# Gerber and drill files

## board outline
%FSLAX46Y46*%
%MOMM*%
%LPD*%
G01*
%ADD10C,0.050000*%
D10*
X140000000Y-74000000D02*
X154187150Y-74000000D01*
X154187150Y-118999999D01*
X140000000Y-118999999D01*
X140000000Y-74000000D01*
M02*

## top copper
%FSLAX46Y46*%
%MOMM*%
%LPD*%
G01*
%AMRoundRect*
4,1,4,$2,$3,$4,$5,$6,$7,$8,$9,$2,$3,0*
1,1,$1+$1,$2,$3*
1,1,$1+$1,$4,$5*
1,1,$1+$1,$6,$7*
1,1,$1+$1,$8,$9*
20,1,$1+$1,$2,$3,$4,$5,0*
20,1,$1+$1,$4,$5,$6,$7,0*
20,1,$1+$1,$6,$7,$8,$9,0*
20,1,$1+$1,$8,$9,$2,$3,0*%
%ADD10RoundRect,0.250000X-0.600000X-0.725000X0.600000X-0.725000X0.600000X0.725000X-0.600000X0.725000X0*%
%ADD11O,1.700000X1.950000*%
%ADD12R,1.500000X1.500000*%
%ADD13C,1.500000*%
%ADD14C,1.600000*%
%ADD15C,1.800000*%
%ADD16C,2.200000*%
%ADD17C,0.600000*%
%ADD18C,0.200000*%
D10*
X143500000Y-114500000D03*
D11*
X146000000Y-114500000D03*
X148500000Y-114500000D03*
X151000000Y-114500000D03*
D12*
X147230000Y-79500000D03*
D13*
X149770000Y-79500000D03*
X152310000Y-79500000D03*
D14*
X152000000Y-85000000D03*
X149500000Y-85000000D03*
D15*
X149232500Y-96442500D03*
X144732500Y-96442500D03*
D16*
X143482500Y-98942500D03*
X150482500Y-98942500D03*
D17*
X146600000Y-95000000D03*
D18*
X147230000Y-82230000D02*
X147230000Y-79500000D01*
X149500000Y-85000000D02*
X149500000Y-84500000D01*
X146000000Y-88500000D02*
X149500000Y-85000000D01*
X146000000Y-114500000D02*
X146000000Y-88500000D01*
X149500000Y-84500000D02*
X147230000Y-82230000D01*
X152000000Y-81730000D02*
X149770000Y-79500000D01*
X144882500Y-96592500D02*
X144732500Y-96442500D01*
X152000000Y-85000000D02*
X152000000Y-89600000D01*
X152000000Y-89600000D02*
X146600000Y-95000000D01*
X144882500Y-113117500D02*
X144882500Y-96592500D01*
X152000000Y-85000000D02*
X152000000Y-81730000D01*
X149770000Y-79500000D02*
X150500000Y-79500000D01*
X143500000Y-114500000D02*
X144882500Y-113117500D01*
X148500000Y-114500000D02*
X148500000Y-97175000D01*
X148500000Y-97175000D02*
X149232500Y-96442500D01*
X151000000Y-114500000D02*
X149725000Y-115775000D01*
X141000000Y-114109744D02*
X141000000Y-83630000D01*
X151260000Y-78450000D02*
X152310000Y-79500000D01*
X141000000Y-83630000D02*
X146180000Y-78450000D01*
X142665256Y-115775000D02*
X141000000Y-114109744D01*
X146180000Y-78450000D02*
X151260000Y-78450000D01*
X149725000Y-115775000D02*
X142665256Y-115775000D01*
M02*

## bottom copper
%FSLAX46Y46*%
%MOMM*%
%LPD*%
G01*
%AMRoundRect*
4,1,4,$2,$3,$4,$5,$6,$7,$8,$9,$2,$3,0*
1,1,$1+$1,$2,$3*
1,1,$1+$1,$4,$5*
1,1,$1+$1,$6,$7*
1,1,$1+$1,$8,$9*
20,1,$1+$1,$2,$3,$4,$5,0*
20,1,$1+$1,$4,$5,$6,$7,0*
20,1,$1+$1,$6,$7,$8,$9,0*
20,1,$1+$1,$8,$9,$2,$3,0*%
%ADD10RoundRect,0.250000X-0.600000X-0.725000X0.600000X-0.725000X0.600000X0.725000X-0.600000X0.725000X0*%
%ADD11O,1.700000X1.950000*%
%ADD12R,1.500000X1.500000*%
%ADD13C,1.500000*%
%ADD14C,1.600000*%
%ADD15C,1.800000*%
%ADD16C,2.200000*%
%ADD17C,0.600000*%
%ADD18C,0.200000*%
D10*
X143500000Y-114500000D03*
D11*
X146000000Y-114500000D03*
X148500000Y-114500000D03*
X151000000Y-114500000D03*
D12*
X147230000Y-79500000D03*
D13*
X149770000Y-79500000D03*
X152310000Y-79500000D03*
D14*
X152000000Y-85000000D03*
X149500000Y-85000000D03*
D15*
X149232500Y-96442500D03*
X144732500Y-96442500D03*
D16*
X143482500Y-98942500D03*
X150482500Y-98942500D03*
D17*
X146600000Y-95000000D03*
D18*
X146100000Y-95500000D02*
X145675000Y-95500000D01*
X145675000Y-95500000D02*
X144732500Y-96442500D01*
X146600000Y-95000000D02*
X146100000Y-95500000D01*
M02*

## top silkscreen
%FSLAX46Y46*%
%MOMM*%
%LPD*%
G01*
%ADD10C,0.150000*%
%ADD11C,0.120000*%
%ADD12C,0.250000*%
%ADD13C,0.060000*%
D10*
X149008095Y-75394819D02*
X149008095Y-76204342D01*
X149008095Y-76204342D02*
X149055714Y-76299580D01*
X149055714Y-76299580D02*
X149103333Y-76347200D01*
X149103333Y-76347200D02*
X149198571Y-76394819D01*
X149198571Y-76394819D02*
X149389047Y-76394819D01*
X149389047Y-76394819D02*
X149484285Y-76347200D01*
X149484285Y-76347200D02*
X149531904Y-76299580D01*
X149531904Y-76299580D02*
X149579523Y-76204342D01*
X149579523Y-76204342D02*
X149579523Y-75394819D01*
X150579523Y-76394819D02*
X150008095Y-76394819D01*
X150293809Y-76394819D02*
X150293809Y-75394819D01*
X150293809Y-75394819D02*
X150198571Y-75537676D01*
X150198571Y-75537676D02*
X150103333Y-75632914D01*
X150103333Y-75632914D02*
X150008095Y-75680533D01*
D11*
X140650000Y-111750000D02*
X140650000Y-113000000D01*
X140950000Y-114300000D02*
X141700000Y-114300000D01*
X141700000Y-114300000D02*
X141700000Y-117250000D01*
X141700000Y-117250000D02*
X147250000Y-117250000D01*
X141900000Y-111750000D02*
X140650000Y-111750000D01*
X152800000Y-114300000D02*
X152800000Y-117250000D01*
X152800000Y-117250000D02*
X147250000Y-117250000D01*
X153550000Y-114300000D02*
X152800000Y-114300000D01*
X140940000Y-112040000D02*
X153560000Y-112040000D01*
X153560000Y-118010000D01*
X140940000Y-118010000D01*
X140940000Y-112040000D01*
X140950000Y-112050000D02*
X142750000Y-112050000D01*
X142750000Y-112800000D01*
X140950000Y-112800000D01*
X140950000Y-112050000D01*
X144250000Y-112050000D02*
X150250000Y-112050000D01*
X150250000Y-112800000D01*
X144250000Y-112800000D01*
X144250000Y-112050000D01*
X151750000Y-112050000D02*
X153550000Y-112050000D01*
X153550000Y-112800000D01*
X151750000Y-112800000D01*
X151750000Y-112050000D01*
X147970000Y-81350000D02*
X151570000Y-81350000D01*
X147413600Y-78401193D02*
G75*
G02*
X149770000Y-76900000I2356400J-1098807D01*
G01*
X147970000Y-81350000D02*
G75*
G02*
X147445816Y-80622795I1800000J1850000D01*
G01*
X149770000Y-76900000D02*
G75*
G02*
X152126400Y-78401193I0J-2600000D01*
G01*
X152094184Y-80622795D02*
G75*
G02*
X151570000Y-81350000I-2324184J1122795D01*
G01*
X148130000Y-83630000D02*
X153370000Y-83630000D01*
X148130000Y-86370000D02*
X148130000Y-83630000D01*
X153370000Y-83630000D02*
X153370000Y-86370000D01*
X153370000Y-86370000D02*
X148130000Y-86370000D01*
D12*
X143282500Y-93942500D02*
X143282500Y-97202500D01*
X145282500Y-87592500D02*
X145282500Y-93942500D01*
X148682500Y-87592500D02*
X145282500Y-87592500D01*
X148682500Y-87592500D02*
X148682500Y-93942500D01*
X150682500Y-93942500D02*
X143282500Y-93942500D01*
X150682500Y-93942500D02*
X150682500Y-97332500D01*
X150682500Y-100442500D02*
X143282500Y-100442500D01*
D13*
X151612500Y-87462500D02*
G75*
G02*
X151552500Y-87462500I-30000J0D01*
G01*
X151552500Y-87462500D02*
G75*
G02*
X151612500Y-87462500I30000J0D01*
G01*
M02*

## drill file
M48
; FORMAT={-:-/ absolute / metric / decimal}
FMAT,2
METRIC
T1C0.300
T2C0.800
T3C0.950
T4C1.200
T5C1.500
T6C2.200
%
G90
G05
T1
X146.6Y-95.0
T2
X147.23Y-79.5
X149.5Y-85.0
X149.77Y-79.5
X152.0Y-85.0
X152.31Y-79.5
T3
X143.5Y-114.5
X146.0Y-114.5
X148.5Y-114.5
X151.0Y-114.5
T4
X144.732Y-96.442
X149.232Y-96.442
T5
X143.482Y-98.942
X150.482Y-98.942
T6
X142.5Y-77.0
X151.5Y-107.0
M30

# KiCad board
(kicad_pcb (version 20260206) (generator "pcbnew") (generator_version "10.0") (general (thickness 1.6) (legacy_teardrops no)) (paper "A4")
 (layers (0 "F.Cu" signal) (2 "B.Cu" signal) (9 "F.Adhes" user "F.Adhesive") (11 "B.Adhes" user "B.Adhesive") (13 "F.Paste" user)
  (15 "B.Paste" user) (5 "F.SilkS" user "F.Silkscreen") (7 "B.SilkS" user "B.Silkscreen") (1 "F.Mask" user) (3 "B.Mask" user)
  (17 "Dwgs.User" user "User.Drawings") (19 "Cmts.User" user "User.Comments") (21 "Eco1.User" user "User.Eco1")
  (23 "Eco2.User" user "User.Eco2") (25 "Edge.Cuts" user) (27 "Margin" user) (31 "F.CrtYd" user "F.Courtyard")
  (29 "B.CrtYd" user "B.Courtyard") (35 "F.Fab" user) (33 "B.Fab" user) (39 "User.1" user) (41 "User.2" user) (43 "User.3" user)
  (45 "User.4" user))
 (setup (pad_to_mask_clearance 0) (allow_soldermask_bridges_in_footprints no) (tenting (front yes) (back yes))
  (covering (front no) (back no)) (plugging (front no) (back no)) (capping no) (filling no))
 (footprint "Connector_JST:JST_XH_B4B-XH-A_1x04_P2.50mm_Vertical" (layer "F.Cu") (at 143.5 114.5)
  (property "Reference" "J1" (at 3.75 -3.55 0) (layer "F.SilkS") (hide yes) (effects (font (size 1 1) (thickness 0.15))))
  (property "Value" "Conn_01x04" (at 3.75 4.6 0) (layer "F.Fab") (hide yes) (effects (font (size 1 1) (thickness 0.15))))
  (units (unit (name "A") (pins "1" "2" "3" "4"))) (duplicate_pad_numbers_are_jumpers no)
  (fp_line (start -2.85 -2.75) (end -2.85 -1.5) (stroke (width 0.12) (type solid)) (layer "F.SilkS"))
  (fp_line (start -2.55 -0.2) (end -1.8 -0.2) (stroke (width 0.12) (type solid)) (layer "F.SilkS"))
  (fp_line (start -1.8 -0.2) (end -1.8 2.75) (stroke (width 0.12) (type solid)) (layer "F.SilkS"))
  (fp_line (start -1.8 2.75) (end 3.75 2.75) (stroke (width 0.12) (type solid)) (layer "F.SilkS"))
  (fp_line (start -1.6 -2.75) (end -2.85 -2.75) (stroke (width 0.12) (type solid)) (layer "F.SilkS"))
  (fp_line (start 9.3 -0.2) (end 9.3 2.75) (stroke (width 0.12) (type solid)) (layer "F.SilkS"))
  (fp_line (start 9.3 2.75) (end 3.75 2.75) (stroke (width 0.12) (type solid)) (layer "F.SilkS"))
  (fp_line (start 10.05 -0.2) (end 9.3 -0.2) (stroke (width 0.12) (type solid)) (layer "F.SilkS"))
  (fp_rect (start -2.56 -2.46) (end 10.06 3.51) (stroke (width 0.12) (type solid)) (fill no) (layer "F.SilkS"))
  (fp_rect (start -2.55 -2.45) (end -0.75 -1.7) (stroke (width 0.12) (type solid)) (fill no) (layer "F.SilkS"))
  (fp_rect (start 0.75 -2.45) (end 6.75 -1.7) (stroke (width 0.12) (type solid)) (fill no) (layer "F.SilkS"))
  (fp_rect (start 8.25 -2.45) (end 10.05 -1.7) (stroke (width 0.12) (type solid)) (fill no) (layer "F.SilkS"))
  (pad "1" thru_hole roundrect (at 0 0) (size 1.7 1.95) (drill 0.95) (layers "*.Cu" "*.Mask") (remove_unused_layers no)
   (roundrect_rratio 0.147059) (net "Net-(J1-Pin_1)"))
  (pad "2" thru_hole oval (at 2.5 0) (size 1.7 1.95) (drill 0.95) (layers "*.Cu" "*.Mask") (remove_unused_layers no) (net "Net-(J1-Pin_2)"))
  (pad "3" thru_hole oval (at 5 0) (size 1.7 1.95) (drill 0.95) (layers "*.Cu" "*.Mask") (remove_unused_layers no) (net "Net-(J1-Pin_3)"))
  (pad "4" thru_hole oval (at 7.5 0) (size 1.7 1.95) (drill 0.95) (layers "*.Cu" "*.Mask") (remove_unused_layers no) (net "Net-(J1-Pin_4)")))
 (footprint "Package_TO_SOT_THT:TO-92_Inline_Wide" (layer "F.Cu") (at 147.23 79.5)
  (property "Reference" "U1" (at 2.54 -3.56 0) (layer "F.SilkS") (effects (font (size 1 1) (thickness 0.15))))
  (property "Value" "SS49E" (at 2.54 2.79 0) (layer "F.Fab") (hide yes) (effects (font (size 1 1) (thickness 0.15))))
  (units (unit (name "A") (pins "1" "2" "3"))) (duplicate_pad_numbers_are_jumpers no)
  (fp_line (start 0.74 1.85) (end 4.34 1.85) (stroke (width 0.12) (type solid)) (layer "F.SilkS"))
  (fp_arc (start 0.1836 -1.098807) (mid 1.143021 -2.192817) (end 2.54 -2.6) (stroke (width 0.12) (type solid)) (layer "F.SilkS"))
  (fp_arc (start 0.74 1.85) (mid 0.446097 1.509328) (end 0.215816 1.122795) (stroke (width 0.12) (type solid)) (layer "F.SilkS"))
  (fp_arc (start 2.54 -2.6) (mid 3.936979 -2.192818) (end 4.8964 -1.098807) (stroke (width 0.12) (type solid)) (layer "F.SilkS"))
  (fp_arc (start 4.864184 1.122795) (mid 4.633903 1.509328) (end 4.34 1.85) (stroke (width 0.12) (type solid)) (layer "F.SilkS"))
  (pad "1" thru_hole rect (at 0 0) (size 1.5 1.5) (drill 0.8) (layers "*.Cu" "*.Mask") (remove_unused_layers no) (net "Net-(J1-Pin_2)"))
  (pad "2" thru_hole circle (at 2.54 0) (size 1.5 1.5) (drill 0.8) (layers "*.Cu" "*.Mask") (remove_unused_layers no) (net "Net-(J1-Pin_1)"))
  (pad "3" thru_hole circle (at 5.08 0) (size 1.5 1.5) (drill 0.8) (layers "*.Cu" "*.Mask") (remove_unused_layers no) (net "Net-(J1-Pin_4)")))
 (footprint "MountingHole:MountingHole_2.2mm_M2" (layer "F.Cu") (at 142.5 77)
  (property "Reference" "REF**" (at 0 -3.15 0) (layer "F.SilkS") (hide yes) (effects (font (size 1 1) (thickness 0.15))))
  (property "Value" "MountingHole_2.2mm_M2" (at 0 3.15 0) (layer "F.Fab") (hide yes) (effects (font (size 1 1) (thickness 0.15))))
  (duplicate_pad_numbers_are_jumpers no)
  (pad "" np_thru_hole circle (at 0 0) (size 2.2 2.2) (drill 2.2) (layers "*.Cu" "*.Mask")))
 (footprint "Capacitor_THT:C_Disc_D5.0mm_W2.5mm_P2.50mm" (layer "F.Cu") (at 152 85 180)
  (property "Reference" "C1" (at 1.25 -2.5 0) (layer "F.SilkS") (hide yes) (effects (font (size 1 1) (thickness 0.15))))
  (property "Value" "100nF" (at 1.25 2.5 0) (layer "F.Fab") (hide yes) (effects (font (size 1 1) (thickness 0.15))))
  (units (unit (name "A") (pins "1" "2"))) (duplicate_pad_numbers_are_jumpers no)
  (fp_line (start 3.87 1.37) (end -1.37 1.37) (stroke (width 0.12) (type solid)) (layer "F.SilkS"))
  (fp_line (start 3.87 -1.37) (end 3.87 1.37) (stroke (width 0.12) (type solid)) (layer "F.SilkS"))
  (fp_line (start -1.37 1.37) (end -1.37 -1.37) (stroke (width 0.12) (type solid)) (layer "F.SilkS"))
  (fp_line (start -1.37 -1.37) (end 3.87 -1.37) (stroke (width 0.12) (type solid)) (layer "F.SilkS"))
  (pad "1" thru_hole circle (at 0 0 180) (size 1.6 1.6) (drill 0.8) (layers "*.Cu" "*.Mask") (remove_unused_layers no)
   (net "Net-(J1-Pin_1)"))
  (pad "2" thru_hole circle (at 2.5 0 180) (size 1.6 1.6) (drill 0.8) (layers "*.Cu" "*.Mask") (remove_unused_layers no)
   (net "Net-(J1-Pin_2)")))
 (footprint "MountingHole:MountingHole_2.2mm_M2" (layer "F.Cu") (at 151.5 107)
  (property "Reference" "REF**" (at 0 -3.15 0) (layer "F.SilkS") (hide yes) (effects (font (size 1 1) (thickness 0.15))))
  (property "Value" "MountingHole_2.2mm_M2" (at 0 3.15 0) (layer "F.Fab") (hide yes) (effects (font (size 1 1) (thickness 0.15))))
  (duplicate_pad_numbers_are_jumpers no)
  (pad "" np_thru_hole circle (at 0 0) (size 2.2 2.2) (drill 2.2) (layers "*.Cu" "*.Mask")))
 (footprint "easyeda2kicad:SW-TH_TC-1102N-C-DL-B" (layer "F.Cu") (at 146.9825 97.6925 180)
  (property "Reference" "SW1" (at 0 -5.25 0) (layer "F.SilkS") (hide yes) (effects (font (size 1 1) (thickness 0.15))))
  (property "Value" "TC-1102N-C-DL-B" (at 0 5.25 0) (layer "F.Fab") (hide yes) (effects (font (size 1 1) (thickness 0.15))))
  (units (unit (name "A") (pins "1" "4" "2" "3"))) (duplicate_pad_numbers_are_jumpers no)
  (fp_line (start 3.7 3.75) (end 3.7 0.49) (stroke (width 0.25) (type solid)) (layer "F.SilkS"))
  (fp_line (start 1.7 10.1) (end 1.7 3.75) (stroke (width 0.25) (type solid)) (layer "F.SilkS"))
  (fp_line (start -1.7 10.1) (end 1.7 10.1) (stroke (width 0.25) (type solid)) (layer "F.SilkS"))
  (fp_line (start -1.7 10.1) (end -1.7 3.75) (stroke (width 0.25) (type solid)) (layer "F.SilkS"))
  (fp_line (start -3.7 3.75) (end 3.7 3.75) (stroke (width 0.25) (type solid)) (layer "F.SilkS"))
  (fp_line (start -3.7 3.75) (end -3.7 0.36) (stroke (width 0.25) (type solid)) (layer "F.SilkS"))
  (fp_line (start -3.7 -2.75) (end 3.7 -2.75) (stroke (width 0.25) (type solid)) (layer "F.SilkS"))
  (fp_circle (center -4.6 10.23) (end -4.57 10.23) (stroke (width 0.06) (type solid)) (fill no) (layer "F.SilkS"))
  (pad "1" thru_hole circle (at -2.25 1.25 180) (size 1.8 1.8) (drill 1.199998) (layers "*.Cu" "*.Mask") (remove_unused_layers no)
   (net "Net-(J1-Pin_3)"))
  (pad "2" thru_hole circle (at 2.25 1.25 180) (size 1.8 1.8) (drill 1.199998) (layers "*.Cu" "*.Mask") (remove_unused_layers no)
   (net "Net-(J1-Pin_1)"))
  (pad "3" thru_hole circle (at 3.5 -1.25 180) (size 2.2 2.2) (drill 1.500022) (layers "*.Cu" "*.Mask") (remove_unused_layers no)
   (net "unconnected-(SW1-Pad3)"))
  (pad "4" thru_hole circle (at -3.5 -1.25 180) (size 2.2 2.2) (drill 1.500022) (layers "*.Cu" "*.Mask") (remove_unused_layers no)
   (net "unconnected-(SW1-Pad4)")))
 (gr_rect (start 140 74) (end 154.18715 118.999999) (stroke (width 0.05) (type default)) (fill no) (layer "Edge.Cuts"))
 (segment (start 147.23 82.23) (end 147.23 79.5) (width 0.2) (layer "F.Cu") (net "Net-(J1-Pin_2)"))
 (segment (start 149.5 85) (end 149.5 84.5) (width 0.2) (layer "F.Cu") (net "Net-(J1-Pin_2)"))
 (segment (start 146 88.5) (end 149.5 85) (width 0.2) (layer "F.Cu") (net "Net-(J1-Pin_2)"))
 (segment (start 146 114.5) (end 146 88.5) (width 0.2) (layer "F.Cu") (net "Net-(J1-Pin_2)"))
 (segment (start 149.5 84.5) (end 147.23 82.23) (width 0.2) (layer "F.Cu") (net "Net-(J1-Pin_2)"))
 (segment (start 152 81.73) (end 149.77 79.5) (width 0.2) (layer "F.Cu") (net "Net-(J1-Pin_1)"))
 (segment (start 144.8825 96.5925) (end 144.7325 96.4425) (width 0.2) (layer "F.Cu") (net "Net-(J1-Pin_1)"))
 (segment (start 152 85) (end 152 89.6) (width 0.2) (layer "F.Cu") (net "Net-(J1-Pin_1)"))
 (segment (start 152 89.6) (end 146.6 95) (width 0.2) (layer "F.Cu") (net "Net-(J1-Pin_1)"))
 (segment (start 144.8825 113.1175) (end 144.8825 96.5925) (width 0.2) (layer "F.Cu") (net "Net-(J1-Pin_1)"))
 (segment (start 152 85) (end 152 81.73) (width 0.2) (layer "F.Cu") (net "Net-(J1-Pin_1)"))
 (segment (start 149.77 79.5) (end 150.5 79.5) (width 0.2) (layer "F.Cu") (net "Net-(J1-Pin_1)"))
 (segment (start 143.5 114.5) (end 144.8825 113.1175) (width 0.2) (layer "F.Cu") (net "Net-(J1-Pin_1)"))
 (via (at 146.6 95) (size 0.6) (drill 0.3) (layers "F.Cu" "B.Cu") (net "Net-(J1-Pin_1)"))
 (segment (start 146.1 95.5) (end 145.675 95.5) (width 0.2) (layer "B.Cu") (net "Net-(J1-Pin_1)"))
 (segment (start 145.675 95.5) (end 144.7325 96.4425) (width 0.2) (layer "B.Cu") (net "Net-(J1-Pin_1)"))
 (segment (start 146.6 95) (end 146.1 95.5) (width 0.2) (layer "B.Cu") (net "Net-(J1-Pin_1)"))
 (segment (start 148.5 114.5) (end 148.5 97.175) (width 0.2) (layer "F.Cu") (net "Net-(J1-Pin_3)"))
 (segment (start 148.5 97.175) (end 149.2325 96.4425) (width 0.2) (layer "F.Cu") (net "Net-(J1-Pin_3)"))
 (segment (start 151 114.5) (end 149.725 115.775) (width 0.2) (layer "F.Cu") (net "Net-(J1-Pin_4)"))
 (segment (start 141 114.109744) (end 141 83.63) (width 0.2) (layer "F.Cu") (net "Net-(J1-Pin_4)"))
 (segment (start 151.26 78.45) (end 152.31 79.5) (width 0.2) (layer "F.Cu") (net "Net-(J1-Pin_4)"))
 (segment (start 141 83.63) (end 146.18 78.45) (width 0.2) (layer "F.Cu") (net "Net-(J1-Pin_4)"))
 (segment (start 142.665256 115.775) (end 141 114.109744) (width 0.2) (layer "F.Cu") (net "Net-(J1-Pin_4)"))
 (segment (start 146.18 78.45) (end 151.26 78.45) (width 0.2) (layer "F.Cu") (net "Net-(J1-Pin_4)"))
 (segment (start 149.725 115.775) (end 142.665256 115.775) (width 0.2) (layer "F.Cu") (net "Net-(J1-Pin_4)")))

